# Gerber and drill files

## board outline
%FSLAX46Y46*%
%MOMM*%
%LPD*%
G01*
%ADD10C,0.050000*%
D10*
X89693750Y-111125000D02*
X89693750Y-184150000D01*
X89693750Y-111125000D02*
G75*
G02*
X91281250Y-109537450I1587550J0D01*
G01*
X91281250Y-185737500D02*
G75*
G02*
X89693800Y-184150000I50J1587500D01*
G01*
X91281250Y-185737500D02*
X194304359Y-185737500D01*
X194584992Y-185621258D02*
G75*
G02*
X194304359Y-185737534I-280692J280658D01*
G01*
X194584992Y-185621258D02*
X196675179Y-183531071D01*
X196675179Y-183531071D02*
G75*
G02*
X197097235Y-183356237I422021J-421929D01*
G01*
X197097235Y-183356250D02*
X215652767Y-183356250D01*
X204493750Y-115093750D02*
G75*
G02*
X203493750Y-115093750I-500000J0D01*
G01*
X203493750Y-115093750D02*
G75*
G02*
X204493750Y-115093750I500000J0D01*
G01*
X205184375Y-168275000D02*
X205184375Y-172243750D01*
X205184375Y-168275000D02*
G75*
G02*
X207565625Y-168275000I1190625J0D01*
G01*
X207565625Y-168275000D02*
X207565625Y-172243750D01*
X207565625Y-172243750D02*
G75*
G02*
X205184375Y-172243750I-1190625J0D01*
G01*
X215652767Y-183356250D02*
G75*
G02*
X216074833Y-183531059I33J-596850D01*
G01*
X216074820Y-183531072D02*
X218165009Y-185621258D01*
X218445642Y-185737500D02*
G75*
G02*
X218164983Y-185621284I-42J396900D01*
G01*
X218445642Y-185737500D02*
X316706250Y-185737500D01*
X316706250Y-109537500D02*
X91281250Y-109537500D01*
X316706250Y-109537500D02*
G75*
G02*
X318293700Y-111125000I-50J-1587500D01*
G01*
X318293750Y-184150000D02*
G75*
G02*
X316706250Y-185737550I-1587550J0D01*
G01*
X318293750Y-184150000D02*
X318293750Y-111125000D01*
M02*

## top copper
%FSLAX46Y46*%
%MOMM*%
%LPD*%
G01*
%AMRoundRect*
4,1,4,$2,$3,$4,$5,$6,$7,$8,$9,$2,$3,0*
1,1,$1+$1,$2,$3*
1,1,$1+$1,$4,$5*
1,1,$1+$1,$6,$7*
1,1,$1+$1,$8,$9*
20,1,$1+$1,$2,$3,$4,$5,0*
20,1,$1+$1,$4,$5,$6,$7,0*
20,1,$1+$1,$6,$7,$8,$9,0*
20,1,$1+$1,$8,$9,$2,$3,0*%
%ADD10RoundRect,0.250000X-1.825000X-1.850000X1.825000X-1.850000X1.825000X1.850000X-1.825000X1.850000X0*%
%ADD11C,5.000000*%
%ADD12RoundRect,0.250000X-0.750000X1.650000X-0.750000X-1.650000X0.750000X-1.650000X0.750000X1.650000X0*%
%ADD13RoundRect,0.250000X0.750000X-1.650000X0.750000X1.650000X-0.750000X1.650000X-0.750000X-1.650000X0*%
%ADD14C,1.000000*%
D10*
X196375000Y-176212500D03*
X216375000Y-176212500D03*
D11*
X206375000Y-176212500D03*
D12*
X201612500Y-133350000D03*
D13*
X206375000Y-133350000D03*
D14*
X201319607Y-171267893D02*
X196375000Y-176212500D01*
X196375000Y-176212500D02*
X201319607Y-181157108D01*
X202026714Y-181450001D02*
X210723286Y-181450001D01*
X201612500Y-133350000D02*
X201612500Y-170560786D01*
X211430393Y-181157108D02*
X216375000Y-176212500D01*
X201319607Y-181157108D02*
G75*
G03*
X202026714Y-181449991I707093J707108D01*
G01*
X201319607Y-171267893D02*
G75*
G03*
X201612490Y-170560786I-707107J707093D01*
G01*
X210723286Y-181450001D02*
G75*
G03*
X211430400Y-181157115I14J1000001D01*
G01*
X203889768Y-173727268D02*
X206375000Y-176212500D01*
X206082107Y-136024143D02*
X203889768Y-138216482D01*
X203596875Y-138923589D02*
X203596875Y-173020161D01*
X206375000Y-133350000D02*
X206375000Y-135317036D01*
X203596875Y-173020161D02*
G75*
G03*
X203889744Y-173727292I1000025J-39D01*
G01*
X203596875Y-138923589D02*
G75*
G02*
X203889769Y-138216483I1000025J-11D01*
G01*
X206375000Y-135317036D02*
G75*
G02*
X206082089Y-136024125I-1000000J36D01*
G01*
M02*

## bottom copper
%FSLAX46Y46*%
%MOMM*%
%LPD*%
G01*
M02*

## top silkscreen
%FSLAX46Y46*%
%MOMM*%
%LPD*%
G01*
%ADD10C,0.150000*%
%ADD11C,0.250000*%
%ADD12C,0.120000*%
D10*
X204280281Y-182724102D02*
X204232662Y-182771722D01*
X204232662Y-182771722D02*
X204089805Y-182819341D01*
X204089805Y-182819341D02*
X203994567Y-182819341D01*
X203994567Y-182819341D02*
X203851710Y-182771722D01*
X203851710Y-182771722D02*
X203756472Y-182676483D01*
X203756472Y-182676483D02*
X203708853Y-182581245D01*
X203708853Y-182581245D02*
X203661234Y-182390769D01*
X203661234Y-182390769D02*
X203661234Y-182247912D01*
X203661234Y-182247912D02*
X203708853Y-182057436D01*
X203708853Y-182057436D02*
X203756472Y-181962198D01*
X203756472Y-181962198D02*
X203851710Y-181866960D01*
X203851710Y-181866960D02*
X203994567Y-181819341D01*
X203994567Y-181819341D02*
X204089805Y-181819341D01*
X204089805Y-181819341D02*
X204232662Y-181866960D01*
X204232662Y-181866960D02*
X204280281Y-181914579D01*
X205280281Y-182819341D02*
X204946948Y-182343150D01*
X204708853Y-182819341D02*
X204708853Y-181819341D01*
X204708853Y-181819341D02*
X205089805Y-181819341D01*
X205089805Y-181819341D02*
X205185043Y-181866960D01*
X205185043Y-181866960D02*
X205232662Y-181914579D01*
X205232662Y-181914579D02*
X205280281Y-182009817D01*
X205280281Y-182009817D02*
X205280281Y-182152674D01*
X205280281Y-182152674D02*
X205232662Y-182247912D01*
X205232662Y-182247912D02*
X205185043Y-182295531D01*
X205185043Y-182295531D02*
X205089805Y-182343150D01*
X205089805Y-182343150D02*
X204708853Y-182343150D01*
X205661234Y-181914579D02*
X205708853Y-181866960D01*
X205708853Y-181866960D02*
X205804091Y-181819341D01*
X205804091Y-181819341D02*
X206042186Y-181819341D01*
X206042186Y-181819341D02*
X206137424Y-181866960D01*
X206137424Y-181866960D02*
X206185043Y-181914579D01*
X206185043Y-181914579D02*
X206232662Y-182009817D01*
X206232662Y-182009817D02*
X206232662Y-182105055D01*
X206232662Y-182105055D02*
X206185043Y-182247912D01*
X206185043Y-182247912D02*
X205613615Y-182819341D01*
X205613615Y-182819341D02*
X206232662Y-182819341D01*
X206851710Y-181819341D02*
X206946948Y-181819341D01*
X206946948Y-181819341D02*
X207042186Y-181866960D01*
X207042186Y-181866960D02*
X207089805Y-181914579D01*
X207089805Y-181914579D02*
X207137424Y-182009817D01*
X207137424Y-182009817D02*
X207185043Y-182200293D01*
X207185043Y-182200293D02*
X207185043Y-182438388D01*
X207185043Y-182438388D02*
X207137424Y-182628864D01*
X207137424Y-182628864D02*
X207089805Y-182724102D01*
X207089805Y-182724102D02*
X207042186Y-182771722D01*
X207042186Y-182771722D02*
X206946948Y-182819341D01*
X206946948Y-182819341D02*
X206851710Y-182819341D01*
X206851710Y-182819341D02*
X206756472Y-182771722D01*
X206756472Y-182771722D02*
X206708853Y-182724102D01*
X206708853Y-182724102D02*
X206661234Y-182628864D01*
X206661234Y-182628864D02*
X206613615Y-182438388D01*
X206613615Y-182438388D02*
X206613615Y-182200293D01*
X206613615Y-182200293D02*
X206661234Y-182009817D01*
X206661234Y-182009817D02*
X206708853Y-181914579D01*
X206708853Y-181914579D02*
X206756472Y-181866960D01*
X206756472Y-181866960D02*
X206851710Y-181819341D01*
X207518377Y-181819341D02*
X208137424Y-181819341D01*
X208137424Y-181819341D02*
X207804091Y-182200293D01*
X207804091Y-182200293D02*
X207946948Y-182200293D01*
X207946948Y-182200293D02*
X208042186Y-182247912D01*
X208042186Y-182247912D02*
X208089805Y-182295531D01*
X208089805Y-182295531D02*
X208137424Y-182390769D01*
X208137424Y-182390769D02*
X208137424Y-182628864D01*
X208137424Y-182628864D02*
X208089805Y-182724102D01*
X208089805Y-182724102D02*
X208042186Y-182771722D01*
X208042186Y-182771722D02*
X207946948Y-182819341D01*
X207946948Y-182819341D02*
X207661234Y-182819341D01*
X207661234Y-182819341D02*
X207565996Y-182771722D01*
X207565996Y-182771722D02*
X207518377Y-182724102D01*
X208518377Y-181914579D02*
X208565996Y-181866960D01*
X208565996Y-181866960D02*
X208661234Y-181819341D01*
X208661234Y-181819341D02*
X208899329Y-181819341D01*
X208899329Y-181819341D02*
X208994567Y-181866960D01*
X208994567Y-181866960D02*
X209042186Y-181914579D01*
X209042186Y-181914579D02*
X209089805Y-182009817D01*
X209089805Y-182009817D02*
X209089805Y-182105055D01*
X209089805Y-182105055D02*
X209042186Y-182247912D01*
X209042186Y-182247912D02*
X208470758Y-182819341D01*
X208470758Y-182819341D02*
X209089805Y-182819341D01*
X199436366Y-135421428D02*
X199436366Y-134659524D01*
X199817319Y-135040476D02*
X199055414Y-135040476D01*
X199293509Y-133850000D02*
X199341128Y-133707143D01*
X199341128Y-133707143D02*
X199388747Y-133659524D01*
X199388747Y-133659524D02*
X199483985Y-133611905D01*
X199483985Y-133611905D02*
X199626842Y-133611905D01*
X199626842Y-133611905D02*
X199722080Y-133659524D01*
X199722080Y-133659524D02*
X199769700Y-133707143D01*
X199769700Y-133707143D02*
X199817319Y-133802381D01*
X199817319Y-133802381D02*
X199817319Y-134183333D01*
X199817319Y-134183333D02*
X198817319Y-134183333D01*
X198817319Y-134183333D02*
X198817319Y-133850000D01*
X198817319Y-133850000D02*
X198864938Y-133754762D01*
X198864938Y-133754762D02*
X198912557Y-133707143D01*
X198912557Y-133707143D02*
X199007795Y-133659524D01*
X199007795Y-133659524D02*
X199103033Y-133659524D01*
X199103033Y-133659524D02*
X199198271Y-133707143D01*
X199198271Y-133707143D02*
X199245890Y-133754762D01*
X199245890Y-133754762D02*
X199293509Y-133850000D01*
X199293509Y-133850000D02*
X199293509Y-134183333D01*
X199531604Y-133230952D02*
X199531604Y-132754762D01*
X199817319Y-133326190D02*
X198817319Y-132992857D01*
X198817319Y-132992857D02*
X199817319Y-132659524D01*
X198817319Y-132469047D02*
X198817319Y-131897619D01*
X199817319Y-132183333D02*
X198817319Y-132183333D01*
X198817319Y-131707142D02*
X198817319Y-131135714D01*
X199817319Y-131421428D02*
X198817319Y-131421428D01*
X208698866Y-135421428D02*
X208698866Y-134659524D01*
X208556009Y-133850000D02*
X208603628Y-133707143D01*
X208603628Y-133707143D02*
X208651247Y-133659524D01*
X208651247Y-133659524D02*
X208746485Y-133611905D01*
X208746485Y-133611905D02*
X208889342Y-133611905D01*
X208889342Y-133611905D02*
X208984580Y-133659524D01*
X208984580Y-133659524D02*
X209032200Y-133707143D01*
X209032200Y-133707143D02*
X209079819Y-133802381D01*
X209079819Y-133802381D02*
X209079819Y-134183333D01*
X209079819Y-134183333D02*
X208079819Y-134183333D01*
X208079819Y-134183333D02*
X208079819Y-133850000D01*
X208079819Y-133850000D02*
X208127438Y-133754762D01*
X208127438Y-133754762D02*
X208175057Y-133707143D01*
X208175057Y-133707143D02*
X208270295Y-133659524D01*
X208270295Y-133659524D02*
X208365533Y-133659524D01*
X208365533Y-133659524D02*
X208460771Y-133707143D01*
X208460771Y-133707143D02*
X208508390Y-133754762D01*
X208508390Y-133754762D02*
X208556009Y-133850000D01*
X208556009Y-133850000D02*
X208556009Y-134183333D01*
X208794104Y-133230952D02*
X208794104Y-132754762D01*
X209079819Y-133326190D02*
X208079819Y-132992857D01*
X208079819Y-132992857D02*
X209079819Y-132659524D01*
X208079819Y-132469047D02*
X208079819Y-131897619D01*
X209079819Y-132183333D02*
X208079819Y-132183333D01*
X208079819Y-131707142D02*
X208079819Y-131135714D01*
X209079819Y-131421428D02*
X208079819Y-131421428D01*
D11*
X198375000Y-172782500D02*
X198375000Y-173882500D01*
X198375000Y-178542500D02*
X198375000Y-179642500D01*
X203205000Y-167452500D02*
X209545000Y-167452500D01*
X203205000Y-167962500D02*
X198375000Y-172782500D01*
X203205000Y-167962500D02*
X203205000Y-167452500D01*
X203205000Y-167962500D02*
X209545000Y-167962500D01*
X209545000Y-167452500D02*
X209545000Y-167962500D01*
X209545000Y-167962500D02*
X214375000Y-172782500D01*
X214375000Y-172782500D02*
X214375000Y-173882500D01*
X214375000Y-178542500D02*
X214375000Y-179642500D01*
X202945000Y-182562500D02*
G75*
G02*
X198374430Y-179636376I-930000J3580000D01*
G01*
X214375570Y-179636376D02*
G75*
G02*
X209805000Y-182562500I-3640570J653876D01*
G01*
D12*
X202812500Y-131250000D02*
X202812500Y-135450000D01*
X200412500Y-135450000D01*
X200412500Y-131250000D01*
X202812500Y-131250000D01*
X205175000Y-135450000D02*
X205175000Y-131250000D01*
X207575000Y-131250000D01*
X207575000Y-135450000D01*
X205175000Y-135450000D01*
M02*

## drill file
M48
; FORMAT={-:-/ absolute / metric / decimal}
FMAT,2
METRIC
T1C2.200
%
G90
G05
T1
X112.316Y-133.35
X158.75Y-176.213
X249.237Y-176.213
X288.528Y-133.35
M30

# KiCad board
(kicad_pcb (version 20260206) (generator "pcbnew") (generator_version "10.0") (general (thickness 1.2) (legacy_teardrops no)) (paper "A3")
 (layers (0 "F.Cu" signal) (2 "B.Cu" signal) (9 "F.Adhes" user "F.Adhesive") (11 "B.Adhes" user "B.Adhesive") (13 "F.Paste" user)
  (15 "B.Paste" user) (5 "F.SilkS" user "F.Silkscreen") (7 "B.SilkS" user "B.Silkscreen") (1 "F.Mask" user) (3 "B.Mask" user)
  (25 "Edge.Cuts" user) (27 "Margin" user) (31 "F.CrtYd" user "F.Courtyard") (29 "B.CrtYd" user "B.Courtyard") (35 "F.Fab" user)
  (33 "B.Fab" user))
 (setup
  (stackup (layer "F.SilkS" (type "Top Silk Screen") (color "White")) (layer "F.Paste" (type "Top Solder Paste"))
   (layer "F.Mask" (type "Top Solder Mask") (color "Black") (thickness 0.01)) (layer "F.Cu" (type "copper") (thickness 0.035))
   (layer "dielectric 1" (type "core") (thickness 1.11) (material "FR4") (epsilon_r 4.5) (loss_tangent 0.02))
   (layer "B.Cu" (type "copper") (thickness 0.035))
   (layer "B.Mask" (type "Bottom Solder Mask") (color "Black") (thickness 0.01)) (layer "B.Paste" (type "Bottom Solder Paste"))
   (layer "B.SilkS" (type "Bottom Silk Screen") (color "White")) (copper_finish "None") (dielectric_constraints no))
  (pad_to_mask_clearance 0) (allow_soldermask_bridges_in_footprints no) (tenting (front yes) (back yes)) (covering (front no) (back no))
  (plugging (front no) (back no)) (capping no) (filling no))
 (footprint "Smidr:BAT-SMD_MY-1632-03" (layer "F.Cu") (at 206.375 176.2125)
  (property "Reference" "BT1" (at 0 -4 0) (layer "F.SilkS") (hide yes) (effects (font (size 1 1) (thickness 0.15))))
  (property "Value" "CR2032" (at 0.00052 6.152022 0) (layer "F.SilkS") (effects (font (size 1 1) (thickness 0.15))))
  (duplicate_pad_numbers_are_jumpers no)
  (fp_line (start -8 -3.43) (end -8 -2.33) (stroke (width 0.25) (type solid)) (layer "F.SilkS"))
  (fp_line (start -8 2.33) (end -8 3.43) (stroke (width 0.25) (type solid)) (layer "F.SilkS"))
  (fp_line (start -3.17 -8.76) (end 3.17 -8.76) (stroke (width 0.25) (type solid)) (layer "F.SilkS"))
  (fp_line (start -3.17 -8.25) (end -8 -3.43) (stroke (width 0.25) (type solid)) (layer "F.SilkS"))
  (fp_line (start -3.17 -8.25) (end -3.17 -8.76) (stroke (width 0.25) (type solid)) (layer "F.SilkS"))
  (fp_line (start -3.17 -8.25) (end 3.17 -8.25) (stroke (width 0.25) (type solid)) (layer "F.SilkS"))
  (fp_line (start 3.17 -8.76) (end 3.17 -8.25) (stroke (width 0.25) (type solid)) (layer "F.SilkS"))
  (fp_line (start 3.17 -8.25) (end 8 -3.43) (stroke (width 0.25) (type solid)) (layer "F.SilkS"))
  (fp_line (start 8 -3.43) (end 8 -2.33) (stroke (width 0.25) (type solid)) (layer "F.SilkS"))
  (fp_line (start 8 2.33) (end 8 3.43) (stroke (width 0.25) (type solid)) (layer "F.SilkS"))
  (fp_arc (start -3.43 6.35) (mid -6.354329 5.885117) (end -8.00057 3.423876) (stroke (width 0.25) (type solid)) (layer "F.SilkS"))
  (fp_arc (start 8.00057 3.423876) (mid 6.354329 5.885117) (end 3.43 6.35) (stroke (width 0.25) (type solid)) (layer "F.SilkS"))
  (pad "1" smd roundrect (at -10 0) (size 4.15 4.2) (layers "F.Cu" "F.Mask" "F.Paste") (roundrect_rratio 0.06024096386) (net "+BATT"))
  (pad "1" smd roundrect (at 10 0) (size 4.15 4.2) (layers "F.Cu" "F.Mask" "F.Paste") (roundrect_rratio 0.06024096386) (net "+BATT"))
  (pad "2" smd circle (at 0 0) (size 5 5) (layers "F.Cu" "F.Mask" "F.Paste") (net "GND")))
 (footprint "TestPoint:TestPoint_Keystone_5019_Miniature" (layer "F.Cu") (at 201.6125 133.35 -90)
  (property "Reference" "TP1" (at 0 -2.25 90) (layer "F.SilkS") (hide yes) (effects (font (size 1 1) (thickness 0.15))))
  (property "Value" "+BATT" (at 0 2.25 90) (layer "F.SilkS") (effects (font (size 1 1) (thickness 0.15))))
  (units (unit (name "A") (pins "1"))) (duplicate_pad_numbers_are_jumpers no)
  (fp_poly (pts (xy -2.1 -1.2) (xy 2.1 -1.2) (xy 2.1 1.2) (xy -2.1 1.2)) (stroke (width 0.12) (type default)) (fill no) (layer "F.SilkS"))
  (pad "1" smd roundrect (at 0 0 270) (size 3.8 2) (layers "F.Cu" "F.Mask" "F.Paste") (roundrect_rratio 0.125) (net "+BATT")))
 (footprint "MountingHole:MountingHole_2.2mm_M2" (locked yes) (layer "F.Cu") (at 112.315625 133.35)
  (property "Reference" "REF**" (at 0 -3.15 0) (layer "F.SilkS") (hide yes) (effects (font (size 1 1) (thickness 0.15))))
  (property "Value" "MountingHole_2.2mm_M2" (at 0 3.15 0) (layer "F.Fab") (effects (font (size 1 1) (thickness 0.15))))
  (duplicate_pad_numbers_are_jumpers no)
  (pad "" np_thru_hole circle (at 0 0) (size 2.2 2.2) (drill 2.2) (layers "*.Cu" "*.Mask")))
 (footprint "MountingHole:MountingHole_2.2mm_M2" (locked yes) (layer "F.Cu") (at 249.2375 176.2125)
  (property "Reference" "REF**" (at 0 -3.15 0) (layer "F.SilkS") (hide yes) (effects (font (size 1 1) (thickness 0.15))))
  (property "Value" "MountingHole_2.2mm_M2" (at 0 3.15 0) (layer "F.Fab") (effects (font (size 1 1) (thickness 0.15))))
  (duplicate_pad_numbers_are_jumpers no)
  (pad "" np_thru_hole circle (at 0 0) (size 2.2 2.2) (drill 2.2) (layers "*.Cu" "*.Mask")))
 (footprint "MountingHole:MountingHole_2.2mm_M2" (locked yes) (layer "F.Cu") (at 158.75 176.2125)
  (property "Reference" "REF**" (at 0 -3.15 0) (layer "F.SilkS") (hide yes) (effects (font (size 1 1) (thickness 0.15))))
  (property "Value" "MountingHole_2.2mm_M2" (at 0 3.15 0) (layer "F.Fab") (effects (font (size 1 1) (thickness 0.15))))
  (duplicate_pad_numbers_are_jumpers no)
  (pad "" np_thru_hole circle (at 0 0) (size 2.2 2.2) (drill 2.2) (layers "*.Cu" "*.Mask")))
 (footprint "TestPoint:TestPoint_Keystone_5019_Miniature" (layer "F.Cu") (at 206.375 133.35 90)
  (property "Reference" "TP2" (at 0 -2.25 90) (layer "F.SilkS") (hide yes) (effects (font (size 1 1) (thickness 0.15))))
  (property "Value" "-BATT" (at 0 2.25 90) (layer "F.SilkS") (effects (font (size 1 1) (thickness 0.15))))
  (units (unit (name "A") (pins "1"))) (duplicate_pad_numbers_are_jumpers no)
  (fp_poly (pts (xy -2.1 -1.2) (xy 2.1 -1.2) (xy 2.1 1.2) (xy -2.1 1.2)) (stroke (width 0.12) (type default)) (fill no) (layer "F.SilkS"))
  (pad "1" smd roundrect (at 0 0 90) (size 3.8 2) (layers "F.Cu" "F.Mask" "F.Paste") (roundrect_rratio 0.125) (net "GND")))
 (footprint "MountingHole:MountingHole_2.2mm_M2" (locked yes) (layer "F.Cu") (at 288.528125 133.35)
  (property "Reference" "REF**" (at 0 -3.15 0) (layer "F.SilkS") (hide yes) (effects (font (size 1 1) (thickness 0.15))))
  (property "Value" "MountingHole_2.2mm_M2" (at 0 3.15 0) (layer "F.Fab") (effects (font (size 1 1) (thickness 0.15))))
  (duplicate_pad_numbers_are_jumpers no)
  (pad "" np_thru_hole circle (at 0 0) (size 2.2 2.2) (drill 2.2) (layers "*.Cu" "*.Mask")))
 (gr_line (start 89.69375 111.125) (end 89.69375 184.15) (stroke (width 0.05) (type default)) (layer "Edge.Cuts"))
 (gr_arc (start 89.69375 111.125) (mid 90.158718 110.002468) (end 91.28125 109.5375) (stroke (width 0.05) (type default))
  (layer "Edge.Cuts"))
 (gr_arc (start 91.28125 185.7375) (mid 90.158718 185.272532) (end 89.69375 184.15) (stroke (width 0.05) (type default)) (layer "Edge.Cuts"))
 (gr_line (start 91.28125 185.7375) (end 194.304359 185.7375) (stroke (width 0.05) (type default)) (layer "Edge.Cuts"))
 (gr_arc (start 194.584992 185.621258) (mid 194.456235 185.707285) (end 194.304359 185.7375) (stroke (width 0.05) (type default))
  (layer "Edge.Cuts"))
 (gr_line (start 194.584992 185.621258) (end 196.675179 183.531071) (stroke (width 0.05) (type default)) (layer "Edge.Cuts"))
 (gr_arc (start 196.675179 183.531071) (mid 196.868817 183.401671) (end 197.097235 183.35625) (stroke (width 0.05) (type default))
  (layer "Edge.Cuts"))
 (gr_line (start 197.097235 183.35625) (end 215.652767 183.35625) (stroke (width 0.05) (type default)) (layer "Edge.Cuts"))
 (gr_circle (center 203.99375 115.09375) (end 204.49375 115.09375) (stroke (width 0.05) (type solid)) (fill no) (layer "Edge.Cuts"))
 (gr_line (start 205.184375 168.275) (end 205.184375 172.24375) (stroke (width 0.05) (type default)) (layer "Edge.Cuts"))
 (gr_arc (start 205.184375 168.275) (mid 206.375 167.084375) (end 207.565625 168.275) (stroke (width 0.05) (type default))
  (layer "Edge.Cuts"))
 (gr_line (start 207.565625 168.275) (end 207.565625 172.24375) (stroke (width 0.05) (type default)) (layer "Edge.Cuts"))
 (gr_arc (start 207.565625 172.24375) (mid 206.375 173.434375) (end 205.184375 172.24375) (stroke (width 0.05) (type default))
  (layer "Edge.Cuts"))
 (gr_arc (start 215.652767 183.35625) (mid 215.881181 183.401685) (end 216.07482 183.531072) (stroke (width 0.05) (type default))
  (layer "Edge.Cuts"))
 (gr_line (start 216.07482 183.531072) (end 218.165009 185.621258) (stroke (width 0.05) (type default)) (layer "Edge.Cuts"))
 (gr_arc (start 218.445642 185.7375) (mid 218.293764 185.70729) (end 218.165009 185.621258) (stroke (width 0.05) (type default))
  (layer "Edge.Cuts"))
 (gr_line (start 218.445642 185.7375) (end 316.70625 185.7375) (stroke (width 0.05) (type default)) (layer "Edge.Cuts"))
 (gr_line (start 316.70625 109.5375) (end 91.28125 109.5375) (stroke (width 0.05) (type default)) (layer "Edge.Cuts"))
 (gr_arc (start 316.70625 109.5375) (mid 317.828782 110.002468) (end 318.29375 111.125) (stroke (width 0.05) (type default))
  (layer "Edge.Cuts"))
 (gr_arc (start 318.29375 184.15) (mid 317.828782 185.272532) (end 316.70625 185.7375) (stroke (width 0.05) (type default))
  (layer "Edge.Cuts"))
 (gr_line (start 318.29375 184.15) (end 318.29375 111.125) (stroke (width 0.05) (type default)) (layer "Edge.Cuts"))
 (segment (start 201.319607 171.267893) (end 196.375 176.2125) (width 1) (layer "F.Cu") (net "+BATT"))
 (segment (start 196.375 176.2125) (end 201.319607 181.157108) (width 1) (layer "F.Cu") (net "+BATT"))
 (segment (start 202.026714 181.450001) (end 210.723286 181.450001) (width 1) (layer "F.Cu") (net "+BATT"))
 (segment (start 201.6125 133.35) (end 201.6125 170.560786) (width 1) (layer "F.Cu") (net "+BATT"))
 (segment (start 211.430393 181.157108) (end 216.375 176.2125) (width 1) (layer "F.Cu") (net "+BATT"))
 (arc (start 201.319607 181.157108) (mid 201.64403 181.373881) (end 202.026714 181.450001) (width 1) (layer "F.Cu") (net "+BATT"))
 (arc (start 201.319607 171.267893) (mid 201.53638 170.94347) (end 201.6125 170.560786) (width 1) (layer "F.Cu") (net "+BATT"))
 (arc (start 210.723286 181.450001) (mid 211.10597 181.373881) (end 211.430393 181.157108) (width 1) (layer "F.Cu") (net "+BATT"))
 (segment (start 203.889768 173.727268) (end 206.375 176.2125) (width 1) (layer "F.Cu") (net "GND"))
 (segment (start 206.082107 136.024143) (end 203.889768 138.216482) (width 1) (layer "F.Cu") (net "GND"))
 (segment (start 203.596875 138.923589) (end 203.596875 173.020161) (width 1) (layer "F.Cu") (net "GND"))
 (segment (start 206.375 133.35) (end 206.375 135.317036) (width 1) (layer "F.Cu") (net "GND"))
 (arc (start 203.596875 173.020161) (mid 203.672995 173.402845) (end 203.889768 173.727268) (width 1) (layer "F.Cu") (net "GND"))
 (arc (start 203.596875 138.923589) (mid 203.672995 138.540905) (end 203.889768 138.216482) (width 1) (layer "F.Cu") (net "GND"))
 (arc (start 206.375 135.317036) (mid 206.29888 135.69972) (end 206.082107 136.024143) (width 1) (layer "F.Cu") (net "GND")))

